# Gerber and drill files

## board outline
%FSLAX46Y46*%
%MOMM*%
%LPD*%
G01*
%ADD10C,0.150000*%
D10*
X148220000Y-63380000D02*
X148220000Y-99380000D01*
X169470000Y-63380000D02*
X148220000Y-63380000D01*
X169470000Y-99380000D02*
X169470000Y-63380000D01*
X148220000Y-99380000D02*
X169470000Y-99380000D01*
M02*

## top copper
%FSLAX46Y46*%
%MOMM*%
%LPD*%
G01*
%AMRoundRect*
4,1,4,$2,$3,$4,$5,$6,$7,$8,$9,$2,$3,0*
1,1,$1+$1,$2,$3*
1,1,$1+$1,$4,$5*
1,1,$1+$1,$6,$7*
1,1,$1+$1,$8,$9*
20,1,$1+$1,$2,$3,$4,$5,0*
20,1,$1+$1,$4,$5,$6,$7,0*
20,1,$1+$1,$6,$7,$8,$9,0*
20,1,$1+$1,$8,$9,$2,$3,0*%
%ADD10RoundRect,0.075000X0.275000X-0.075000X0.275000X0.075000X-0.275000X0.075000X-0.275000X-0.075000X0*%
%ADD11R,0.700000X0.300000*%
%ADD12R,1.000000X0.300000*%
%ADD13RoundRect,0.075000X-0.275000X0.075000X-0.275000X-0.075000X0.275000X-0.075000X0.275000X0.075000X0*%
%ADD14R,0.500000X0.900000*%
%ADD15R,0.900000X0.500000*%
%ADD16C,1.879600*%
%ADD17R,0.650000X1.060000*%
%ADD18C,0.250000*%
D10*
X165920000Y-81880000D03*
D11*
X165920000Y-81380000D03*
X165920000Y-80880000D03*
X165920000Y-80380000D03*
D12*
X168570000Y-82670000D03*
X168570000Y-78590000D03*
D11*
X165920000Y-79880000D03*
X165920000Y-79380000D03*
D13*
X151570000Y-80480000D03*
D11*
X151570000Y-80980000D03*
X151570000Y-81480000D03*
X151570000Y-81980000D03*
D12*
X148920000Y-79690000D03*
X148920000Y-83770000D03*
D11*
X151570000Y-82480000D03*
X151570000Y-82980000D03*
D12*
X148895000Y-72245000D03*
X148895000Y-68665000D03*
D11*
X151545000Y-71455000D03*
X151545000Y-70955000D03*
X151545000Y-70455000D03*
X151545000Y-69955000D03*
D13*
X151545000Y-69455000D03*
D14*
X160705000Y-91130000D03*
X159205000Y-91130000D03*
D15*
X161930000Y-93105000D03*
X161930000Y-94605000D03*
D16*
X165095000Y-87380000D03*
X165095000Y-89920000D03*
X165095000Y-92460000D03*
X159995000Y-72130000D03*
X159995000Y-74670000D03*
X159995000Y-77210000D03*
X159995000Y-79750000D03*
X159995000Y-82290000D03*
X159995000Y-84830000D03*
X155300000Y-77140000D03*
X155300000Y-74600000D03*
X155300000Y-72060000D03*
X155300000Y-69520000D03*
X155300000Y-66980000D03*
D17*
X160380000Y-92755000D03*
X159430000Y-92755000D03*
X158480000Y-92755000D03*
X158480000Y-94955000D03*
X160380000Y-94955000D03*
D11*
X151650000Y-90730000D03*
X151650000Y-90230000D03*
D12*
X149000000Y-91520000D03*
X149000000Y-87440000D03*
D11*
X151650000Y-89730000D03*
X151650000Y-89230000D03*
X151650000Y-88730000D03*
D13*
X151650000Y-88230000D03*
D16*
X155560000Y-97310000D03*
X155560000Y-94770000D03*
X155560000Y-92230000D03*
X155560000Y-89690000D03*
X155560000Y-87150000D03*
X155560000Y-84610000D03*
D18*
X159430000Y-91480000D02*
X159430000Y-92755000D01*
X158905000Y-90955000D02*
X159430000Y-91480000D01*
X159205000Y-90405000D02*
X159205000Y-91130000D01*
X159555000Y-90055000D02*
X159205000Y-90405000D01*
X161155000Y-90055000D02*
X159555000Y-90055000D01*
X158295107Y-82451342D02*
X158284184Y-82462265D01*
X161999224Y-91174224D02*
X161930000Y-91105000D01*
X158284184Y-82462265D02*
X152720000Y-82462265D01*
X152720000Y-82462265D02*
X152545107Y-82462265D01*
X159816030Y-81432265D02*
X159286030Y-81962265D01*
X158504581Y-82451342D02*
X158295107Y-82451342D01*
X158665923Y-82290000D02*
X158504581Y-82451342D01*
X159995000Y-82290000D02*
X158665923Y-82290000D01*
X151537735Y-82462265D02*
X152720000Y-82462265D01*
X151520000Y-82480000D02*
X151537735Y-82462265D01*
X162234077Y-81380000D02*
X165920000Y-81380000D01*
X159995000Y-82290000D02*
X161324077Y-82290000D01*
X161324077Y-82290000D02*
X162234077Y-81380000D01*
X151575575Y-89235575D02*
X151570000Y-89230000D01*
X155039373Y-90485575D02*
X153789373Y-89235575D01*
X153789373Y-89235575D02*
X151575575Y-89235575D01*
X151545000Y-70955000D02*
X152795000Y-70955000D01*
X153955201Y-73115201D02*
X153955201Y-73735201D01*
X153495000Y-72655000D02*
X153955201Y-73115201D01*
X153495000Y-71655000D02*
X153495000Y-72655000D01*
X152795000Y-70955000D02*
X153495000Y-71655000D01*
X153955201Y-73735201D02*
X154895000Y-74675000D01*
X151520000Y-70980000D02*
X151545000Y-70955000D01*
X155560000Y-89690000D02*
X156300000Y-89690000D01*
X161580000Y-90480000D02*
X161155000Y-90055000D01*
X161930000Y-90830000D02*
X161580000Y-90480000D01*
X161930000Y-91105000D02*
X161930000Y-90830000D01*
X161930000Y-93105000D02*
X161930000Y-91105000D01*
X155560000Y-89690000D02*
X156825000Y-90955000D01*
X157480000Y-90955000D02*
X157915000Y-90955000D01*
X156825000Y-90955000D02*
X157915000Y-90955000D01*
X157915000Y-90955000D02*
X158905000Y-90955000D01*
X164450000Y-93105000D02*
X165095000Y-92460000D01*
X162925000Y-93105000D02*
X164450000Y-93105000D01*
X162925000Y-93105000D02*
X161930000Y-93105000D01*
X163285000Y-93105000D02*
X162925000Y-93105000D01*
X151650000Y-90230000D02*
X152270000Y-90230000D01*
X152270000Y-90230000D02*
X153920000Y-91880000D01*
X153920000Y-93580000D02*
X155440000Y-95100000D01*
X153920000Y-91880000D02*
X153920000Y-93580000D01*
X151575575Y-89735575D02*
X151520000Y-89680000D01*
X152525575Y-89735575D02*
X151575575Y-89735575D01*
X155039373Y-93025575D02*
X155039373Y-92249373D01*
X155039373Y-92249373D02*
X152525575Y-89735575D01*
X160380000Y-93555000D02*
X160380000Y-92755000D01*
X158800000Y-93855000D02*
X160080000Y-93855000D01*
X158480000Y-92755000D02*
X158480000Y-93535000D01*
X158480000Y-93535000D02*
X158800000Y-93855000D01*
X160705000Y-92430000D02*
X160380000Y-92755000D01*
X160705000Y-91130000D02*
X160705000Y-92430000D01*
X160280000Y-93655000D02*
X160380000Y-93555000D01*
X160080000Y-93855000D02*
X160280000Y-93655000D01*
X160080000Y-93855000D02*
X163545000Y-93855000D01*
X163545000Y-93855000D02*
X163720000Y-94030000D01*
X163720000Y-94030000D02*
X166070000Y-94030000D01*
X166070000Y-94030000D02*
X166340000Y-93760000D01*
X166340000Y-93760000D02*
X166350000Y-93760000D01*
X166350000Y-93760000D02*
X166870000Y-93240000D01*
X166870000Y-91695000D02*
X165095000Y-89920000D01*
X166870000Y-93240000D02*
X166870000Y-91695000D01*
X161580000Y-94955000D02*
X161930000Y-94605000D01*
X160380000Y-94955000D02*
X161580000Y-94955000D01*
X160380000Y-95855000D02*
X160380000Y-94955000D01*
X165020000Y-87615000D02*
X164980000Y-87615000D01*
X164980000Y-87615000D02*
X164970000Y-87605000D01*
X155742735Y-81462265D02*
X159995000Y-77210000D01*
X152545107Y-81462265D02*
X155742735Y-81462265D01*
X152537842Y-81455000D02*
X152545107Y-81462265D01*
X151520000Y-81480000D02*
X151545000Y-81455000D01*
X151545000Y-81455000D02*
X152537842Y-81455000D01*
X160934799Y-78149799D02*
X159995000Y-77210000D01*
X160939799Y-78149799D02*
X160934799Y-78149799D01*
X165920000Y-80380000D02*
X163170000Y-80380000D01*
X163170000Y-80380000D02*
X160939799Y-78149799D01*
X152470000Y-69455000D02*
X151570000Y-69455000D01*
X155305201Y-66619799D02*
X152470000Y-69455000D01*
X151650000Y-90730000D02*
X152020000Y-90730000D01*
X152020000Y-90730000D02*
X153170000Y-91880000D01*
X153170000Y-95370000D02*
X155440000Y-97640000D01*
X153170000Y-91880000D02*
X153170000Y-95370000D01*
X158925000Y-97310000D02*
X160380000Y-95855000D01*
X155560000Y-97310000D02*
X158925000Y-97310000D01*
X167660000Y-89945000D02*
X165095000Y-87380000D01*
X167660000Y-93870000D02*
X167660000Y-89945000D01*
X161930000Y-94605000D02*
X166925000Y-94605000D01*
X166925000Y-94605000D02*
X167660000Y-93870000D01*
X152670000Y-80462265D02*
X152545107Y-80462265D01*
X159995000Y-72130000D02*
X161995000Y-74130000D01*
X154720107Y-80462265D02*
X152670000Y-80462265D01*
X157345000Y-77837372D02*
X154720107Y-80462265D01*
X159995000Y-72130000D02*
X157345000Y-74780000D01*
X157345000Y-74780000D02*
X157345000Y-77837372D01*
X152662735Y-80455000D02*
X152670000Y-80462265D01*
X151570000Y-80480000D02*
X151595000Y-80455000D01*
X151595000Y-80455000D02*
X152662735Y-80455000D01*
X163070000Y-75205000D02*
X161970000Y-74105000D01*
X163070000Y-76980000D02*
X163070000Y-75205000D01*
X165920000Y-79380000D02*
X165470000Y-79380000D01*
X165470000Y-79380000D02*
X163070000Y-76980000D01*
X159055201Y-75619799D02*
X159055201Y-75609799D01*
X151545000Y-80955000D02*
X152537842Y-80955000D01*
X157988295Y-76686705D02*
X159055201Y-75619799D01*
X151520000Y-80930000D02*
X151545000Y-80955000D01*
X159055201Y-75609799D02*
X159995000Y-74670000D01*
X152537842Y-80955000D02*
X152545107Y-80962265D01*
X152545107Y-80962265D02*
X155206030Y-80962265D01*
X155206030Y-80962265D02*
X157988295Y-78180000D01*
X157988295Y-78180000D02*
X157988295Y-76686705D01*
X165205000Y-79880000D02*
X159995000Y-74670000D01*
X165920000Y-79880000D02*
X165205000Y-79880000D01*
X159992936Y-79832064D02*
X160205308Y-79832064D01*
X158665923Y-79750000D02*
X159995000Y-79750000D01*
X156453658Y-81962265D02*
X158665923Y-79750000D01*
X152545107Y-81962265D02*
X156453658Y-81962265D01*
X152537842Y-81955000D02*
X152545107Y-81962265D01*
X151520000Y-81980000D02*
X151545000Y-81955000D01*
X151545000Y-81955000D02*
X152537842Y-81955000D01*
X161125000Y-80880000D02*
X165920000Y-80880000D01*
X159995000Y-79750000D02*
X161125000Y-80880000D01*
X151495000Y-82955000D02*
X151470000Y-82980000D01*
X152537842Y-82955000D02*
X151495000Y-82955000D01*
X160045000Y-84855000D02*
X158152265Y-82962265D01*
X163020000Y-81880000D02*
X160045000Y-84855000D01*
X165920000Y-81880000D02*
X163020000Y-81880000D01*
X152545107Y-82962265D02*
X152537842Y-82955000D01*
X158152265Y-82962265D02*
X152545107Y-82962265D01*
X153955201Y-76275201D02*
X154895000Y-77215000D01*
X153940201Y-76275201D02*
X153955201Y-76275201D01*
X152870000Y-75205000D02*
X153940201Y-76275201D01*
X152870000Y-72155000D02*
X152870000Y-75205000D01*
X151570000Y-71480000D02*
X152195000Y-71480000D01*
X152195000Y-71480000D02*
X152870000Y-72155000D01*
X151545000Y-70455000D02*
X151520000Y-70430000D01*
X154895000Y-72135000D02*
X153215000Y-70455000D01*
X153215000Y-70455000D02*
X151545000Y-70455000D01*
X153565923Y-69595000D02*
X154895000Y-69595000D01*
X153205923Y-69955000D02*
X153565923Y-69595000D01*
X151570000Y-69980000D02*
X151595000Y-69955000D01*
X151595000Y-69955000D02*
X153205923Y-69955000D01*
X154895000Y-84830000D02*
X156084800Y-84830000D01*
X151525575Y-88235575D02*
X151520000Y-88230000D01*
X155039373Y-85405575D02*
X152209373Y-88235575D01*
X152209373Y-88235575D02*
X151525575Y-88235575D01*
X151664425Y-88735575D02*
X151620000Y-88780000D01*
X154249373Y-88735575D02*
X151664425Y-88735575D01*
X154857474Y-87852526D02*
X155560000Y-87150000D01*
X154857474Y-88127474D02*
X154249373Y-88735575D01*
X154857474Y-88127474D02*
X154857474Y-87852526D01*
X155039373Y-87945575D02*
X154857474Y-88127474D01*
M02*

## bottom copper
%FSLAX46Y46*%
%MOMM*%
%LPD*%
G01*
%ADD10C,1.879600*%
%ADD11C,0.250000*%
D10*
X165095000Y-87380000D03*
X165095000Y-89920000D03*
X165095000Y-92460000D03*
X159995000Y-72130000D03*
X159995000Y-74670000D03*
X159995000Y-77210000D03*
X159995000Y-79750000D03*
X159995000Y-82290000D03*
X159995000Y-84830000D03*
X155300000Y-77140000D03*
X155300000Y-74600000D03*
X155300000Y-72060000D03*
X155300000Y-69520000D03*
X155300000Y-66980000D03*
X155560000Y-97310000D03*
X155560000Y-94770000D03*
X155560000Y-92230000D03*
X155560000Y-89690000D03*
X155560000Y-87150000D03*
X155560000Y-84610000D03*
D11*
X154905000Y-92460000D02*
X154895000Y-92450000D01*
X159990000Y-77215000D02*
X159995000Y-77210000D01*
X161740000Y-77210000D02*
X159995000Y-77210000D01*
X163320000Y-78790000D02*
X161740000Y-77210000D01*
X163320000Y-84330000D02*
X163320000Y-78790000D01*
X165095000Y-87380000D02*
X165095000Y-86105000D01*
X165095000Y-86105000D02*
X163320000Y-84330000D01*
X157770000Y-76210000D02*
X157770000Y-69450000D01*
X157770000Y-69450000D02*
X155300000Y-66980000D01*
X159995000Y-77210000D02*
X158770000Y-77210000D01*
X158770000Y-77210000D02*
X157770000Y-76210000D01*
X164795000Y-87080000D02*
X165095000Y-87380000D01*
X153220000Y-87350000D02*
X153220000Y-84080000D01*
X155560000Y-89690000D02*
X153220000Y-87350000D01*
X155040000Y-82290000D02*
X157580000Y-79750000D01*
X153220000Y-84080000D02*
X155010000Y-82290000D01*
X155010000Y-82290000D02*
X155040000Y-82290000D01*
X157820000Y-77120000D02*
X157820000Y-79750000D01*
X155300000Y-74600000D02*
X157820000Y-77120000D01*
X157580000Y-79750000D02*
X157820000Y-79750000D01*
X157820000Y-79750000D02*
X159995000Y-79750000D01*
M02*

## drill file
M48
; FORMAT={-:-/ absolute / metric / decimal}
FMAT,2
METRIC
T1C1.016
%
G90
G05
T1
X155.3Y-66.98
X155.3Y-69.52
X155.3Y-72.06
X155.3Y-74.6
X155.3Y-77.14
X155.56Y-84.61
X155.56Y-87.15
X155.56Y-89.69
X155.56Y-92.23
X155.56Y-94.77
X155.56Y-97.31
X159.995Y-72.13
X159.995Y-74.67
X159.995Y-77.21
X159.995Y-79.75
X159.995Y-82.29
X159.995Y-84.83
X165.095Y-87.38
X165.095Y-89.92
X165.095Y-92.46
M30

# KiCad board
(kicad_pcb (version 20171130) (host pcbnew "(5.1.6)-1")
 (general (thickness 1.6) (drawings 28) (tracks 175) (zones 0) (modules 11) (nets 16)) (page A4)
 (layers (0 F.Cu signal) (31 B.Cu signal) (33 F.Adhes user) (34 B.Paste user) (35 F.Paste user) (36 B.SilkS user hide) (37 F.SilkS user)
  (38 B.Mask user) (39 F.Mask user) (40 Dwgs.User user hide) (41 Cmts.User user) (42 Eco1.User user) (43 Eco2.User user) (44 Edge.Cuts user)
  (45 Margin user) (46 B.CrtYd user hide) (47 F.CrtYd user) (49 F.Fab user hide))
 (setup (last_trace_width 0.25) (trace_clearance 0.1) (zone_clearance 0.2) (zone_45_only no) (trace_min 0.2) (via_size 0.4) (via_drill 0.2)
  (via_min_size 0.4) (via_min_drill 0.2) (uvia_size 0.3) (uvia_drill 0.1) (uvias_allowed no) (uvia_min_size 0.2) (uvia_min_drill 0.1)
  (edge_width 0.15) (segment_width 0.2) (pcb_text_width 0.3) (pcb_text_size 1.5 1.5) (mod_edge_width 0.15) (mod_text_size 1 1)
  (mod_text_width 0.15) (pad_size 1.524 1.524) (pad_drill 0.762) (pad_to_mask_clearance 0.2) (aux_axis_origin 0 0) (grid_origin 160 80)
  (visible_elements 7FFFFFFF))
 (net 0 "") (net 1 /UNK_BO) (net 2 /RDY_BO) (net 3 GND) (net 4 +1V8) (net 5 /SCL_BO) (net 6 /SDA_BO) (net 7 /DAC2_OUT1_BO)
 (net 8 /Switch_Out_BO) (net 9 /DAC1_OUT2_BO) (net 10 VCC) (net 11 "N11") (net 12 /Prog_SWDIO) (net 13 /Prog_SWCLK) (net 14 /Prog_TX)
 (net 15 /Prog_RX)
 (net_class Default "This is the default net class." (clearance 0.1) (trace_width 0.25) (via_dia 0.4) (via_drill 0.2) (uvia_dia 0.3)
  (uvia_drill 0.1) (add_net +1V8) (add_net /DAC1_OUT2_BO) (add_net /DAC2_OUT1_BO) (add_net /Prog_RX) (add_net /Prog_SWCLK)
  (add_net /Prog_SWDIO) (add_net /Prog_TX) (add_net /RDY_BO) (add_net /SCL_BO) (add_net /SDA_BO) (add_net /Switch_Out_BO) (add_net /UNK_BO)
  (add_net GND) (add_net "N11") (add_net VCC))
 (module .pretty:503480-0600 (layer F.Cu) (at 165.92 80.63 90) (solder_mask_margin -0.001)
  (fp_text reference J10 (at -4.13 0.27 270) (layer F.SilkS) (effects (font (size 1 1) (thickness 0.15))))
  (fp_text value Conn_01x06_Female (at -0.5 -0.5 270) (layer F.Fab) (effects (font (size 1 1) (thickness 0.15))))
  (pad 1 smd roundrect (at -1.25 0 90) (size 0.3 0.7) (layers F.Cu F.Paste F.Mask) (roundrect_rratio 0.25) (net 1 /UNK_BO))
  (pad 2 smd rect (at -0.75 0 90) (size 0.3 0.7) (layers F.Cu F.Paste F.Mask) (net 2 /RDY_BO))
  (pad 3 smd rect (at -0.25 0 90) (size 0.3 0.7) (layers F.Cu F.Paste F.Mask) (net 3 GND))
  (pad 4 smd rect (at 0.25 0 90) (size 0.3 0.7) (layers F.Cu F.Paste F.Mask) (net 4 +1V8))
  (pad 0 smd rect (at -2.04 2.65 90) (size 0.3 1) (layers F.Cu F.Paste F.Mask))
  (pad 0 smd rect (at 2.04 2.65 90) (size 0.3 1) (layers F.Cu F.Paste F.Mask))
  (pad 5 smd rect (at 0.75 0 90) (size 0.3 0.7) (layers F.Cu F.Paste F.Mask) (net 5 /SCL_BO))
  (pad 6 smd rect (at 1.25 0 90) (size 0.3 0.7) (layers F.Cu F.Paste F.Mask) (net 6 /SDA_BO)))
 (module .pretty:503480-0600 (layer F.Cu) (at 151.57 81.73 270) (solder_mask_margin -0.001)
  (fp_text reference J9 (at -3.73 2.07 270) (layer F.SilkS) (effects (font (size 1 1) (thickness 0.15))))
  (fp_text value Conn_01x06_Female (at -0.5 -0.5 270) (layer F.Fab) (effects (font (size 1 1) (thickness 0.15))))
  (pad 1 smd roundrect (at -1.25 0 270) (size 0.3 0.7) (layers F.Cu F.Paste F.Mask) (roundrect_rratio 0.25) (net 6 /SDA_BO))
  (pad 2 smd rect (at -0.75 0 270) (size 0.3 0.7) (layers F.Cu F.Paste F.Mask) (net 5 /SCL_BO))
  (pad 3 smd rect (at -0.25 0 270) (size 0.3 0.7) (layers F.Cu F.Paste F.Mask) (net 4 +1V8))
  (pad 4 smd rect (at 0.25 0 270) (size 0.3 0.7) (layers F.Cu F.Paste F.Mask) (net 3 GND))
  (pad 0 smd rect (at -2.04 2.65 270) (size 0.3 1) (layers F.Cu F.Paste F.Mask))
  (pad 0 smd rect (at 2.04 2.65 270) (size 0.3 1) (layers F.Cu F.Paste F.Mask))
  (pad 5 smd rect (at 0.75 0 270) (size 0.3 0.7) (layers F.Cu F.Paste F.Mask) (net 2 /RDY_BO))
  (pad 6 smd rect (at 1.25 0 270) (size 0.3 0.7) (layers F.Cu F.Paste F.Mask) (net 1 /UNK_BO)))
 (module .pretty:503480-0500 (layer F.Cu) (at 151.545 70.455 270) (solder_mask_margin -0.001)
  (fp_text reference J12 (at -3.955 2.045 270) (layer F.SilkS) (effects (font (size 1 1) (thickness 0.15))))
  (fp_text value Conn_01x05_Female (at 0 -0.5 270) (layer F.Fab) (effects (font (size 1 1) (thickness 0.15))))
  (pad 0 smd rect (at 1.79 2.65 270) (size 0.3 1) (layers F.Cu F.Paste F.Mask))
  (pad 0 smd rect (at -1.79 2.65 270) (size 0.3 1) (layers F.Cu F.Paste F.Mask))
  (pad 5 smd rect (at 1 0 270) (size 0.3 0.7) (layers F.Cu F.Paste F.Mask) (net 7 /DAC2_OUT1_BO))
  (pad 4 smd rect (at 0.5 0 270) (size 0.3 0.7) (layers F.Cu F.Paste F.Mask) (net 3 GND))
  (pad 3 smd rect (at 0 0 270) (size 0.3 0.7) (layers F.Cu F.Paste F.Mask) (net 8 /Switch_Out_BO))
  (pad 2 smd rect (at -0.5 0 270) (size 0.3 0.7) (layers F.Cu F.Paste F.Mask) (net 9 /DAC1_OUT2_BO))
  (pad 1 smd roundrect (at -1 0 270) (size 0.3 0.7) (layers F.Cu F.Paste F.Mask) (roundrect_rratio 0.25) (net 4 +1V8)))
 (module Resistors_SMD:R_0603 (layer F.Cu) (at 159.955 91.13)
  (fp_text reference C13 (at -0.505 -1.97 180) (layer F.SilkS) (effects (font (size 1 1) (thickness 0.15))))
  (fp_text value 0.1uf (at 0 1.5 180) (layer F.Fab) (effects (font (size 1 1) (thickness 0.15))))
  (pad 2 smd rect (at 0.75 0) (size 0.5 0.9) (layers F.Cu F.Paste F.Mask) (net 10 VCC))
  (pad 1 smd rect (at -0.75 0) (size 0.5 0.9) (layers F.Cu F.Paste F.Mask) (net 3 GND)))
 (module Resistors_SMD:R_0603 (layer F.Cu) (at 161.93 93.855 270)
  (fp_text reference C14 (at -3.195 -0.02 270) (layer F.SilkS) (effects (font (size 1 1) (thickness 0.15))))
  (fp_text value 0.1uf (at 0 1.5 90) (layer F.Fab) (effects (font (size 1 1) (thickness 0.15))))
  (pad 1 smd rect (at -0.75 0 270) (size 0.5 0.9) (layers F.Cu F.Paste F.Mask) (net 3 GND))
  (pad 2 smd rect (at 0.75 0 270) (size 0.5 0.9) (layers F.Cu F.Paste F.Mask) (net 4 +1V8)))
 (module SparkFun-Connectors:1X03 (layer F.Cu) (at 165.095 87.38 270)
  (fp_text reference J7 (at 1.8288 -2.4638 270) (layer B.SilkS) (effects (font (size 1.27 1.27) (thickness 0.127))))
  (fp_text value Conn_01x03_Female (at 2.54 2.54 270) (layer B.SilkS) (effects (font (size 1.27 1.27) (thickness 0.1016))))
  (pad 1 thru_hole circle (at 0 0 270) (size 1.8796 1.8796) (drill 1.016) (layers F&B.Cu F.Paste F.SilkS F.Mask) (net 4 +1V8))
  (pad 2 thru_hole circle (at 2.54 0 270) (size 1.8796 1.8796) (drill 1.016) (layers F&B.Cu F.Paste F.SilkS F.Mask) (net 10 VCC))
  (pad 3 thru_hole circle (at 5.08 0 270) (size 1.8796 1.8796) (drill 1.016) (layers F&B.Cu F.Paste F.SilkS F.Mask) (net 3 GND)))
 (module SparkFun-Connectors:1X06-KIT (layer F.Cu) (at 159.995 72.13 270)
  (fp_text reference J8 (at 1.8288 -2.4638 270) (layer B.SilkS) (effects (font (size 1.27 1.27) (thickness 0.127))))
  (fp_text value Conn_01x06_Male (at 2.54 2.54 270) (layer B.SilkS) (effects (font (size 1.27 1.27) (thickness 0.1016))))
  (pad 1 thru_hole circle (at 0 0 270) (size 1.8796 1.8796) (drill 1.016) (layers F&B.Cu F.Paste F.SilkS F.Mask) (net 6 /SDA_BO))
  (pad 2 thru_hole circle (at 2.54 0 270) (size 1.8796 1.8796) (drill 1.016) (layers F&B.Cu F.Paste F.SilkS F.Mask) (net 5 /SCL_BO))
  (pad 3 thru_hole circle (at 5.08 0 270) (size 1.8796 1.8796) (drill 1.016) (layers F&B.Cu F.Paste F.SilkS F.Mask) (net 4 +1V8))
  (pad 4 thru_hole circle (at 7.62 0 270) (size 1.8796 1.8796) (drill 1.016) (layers F&B.Cu F.Paste F.SilkS F.Mask) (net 3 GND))
  (pad 5 thru_hole circle (at 10.16 0 270) (size 1.8796 1.8796) (drill 1.016) (layers F&B.Cu F.Paste F.SilkS F.Mask) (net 2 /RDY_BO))
  (pad 6 thru_hole circle (at 12.7 0 270) (size 1.8796 1.8796) (drill 1.016) (layers F&B.Cu F.Paste F.SilkS F.Mask) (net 1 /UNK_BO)))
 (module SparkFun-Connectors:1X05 (layer F.Cu) (at 155.3 77.14 90)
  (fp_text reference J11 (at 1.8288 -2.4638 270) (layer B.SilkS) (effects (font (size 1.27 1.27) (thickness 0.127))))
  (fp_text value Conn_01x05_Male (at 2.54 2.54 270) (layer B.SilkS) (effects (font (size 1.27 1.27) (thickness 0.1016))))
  (pad 1 thru_hole circle (at 0 0 90) (size 1.8796 1.8796) (drill 1.016) (layers F&B.Cu F.Paste F.SilkS F.Mask) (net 7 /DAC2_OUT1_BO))
  (pad 2 thru_hole circle (at 2.54 0 90) (size 1.8796 1.8796) (drill 1.016) (layers F&B.Cu F.Paste F.SilkS F.Mask) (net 3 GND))
  (pad 3 thru_hole circle (at 5.08 0 90) (size 1.8796 1.8796) (drill 1.016) (layers F&B.Cu F.Paste F.SilkS F.Mask) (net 8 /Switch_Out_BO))
  (pad 4 thru_hole circle (at 7.62 0 90) (size 1.8796 1.8796) (drill 1.016) (layers F&B.Cu F.Paste F.SilkS F.Mask) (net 9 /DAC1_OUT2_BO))
  (pad 5 thru_hole circle (at 10.16 0 90) (size 1.8796 1.8796) (drill 1.016) (layers F&B.Cu F.Paste F.SilkS F.Mask) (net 4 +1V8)))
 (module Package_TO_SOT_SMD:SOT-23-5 (layer F.Cu) (at 159.43 93.855 270) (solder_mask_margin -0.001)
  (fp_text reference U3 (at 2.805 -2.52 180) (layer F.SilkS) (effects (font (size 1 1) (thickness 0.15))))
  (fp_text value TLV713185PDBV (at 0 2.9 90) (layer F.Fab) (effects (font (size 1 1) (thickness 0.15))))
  (pad 1 smd rect (at -1.1 -0.95 270) (size 1.06 0.65) (layers F.Cu F.Paste F.Mask) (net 10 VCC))
  (pad 2 smd rect (at -1.1 0 270) (size 1.06 0.65) (layers F.Cu F.Paste F.Mask) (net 3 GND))
  (pad 3 smd rect (at -1.1 0.95 270) (size 1.06 0.65) (layers F.Cu F.Paste F.Mask) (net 10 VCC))
  (pad 4 smd rect (at 1.1 0.95 270) (size 1.06 0.65) (layers F.Cu F.Paste F.Mask) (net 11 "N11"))
  (pad 5 smd rect (at 1.1 -0.95 270) (size 1.06 0.65) (layers F.Cu F.Paste F.Mask) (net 4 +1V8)))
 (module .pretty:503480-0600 (layer F.Cu) (at 151.65 89.48 270) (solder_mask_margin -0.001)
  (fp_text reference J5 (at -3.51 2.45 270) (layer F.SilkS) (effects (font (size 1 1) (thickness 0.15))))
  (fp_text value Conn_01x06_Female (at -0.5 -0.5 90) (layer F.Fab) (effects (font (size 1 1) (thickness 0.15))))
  (pad 6 smd rect (at 1.25 0 270) (size 0.3 0.7) (layers F.Cu F.Paste F.Mask) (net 4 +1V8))
  (pad 5 smd rect (at 0.75 0 270) (size 0.3 0.7) (layers F.Cu F.Paste F.Mask) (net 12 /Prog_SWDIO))
  (pad 0 smd rect (at 2.04 2.65 270) (size 0.3 1) (layers F.Cu F.Paste F.Mask))
  (pad 0 smd rect (at -2.04 2.65 270) (size 0.3 1) (layers F.Cu F.Paste F.Mask))
  (pad 4 smd rect (at 0.25 0 270) (size 0.3 0.7) (layers F.Cu F.Paste F.Mask) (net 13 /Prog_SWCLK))
  (pad 3 smd rect (at -0.25 0 270) (size 0.3 0.7) (layers F.Cu F.Paste F.Mask) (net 3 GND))
  (pad 2 smd rect (at -0.75 0 270) (size 0.3 0.7) (layers F.Cu F.Paste F.Mask) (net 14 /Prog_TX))
  (pad 1 smd roundrect (at -1.25 0 270) (size 0.3 0.7) (layers F.Cu F.Paste F.Mask) (roundrect_rratio 0.25) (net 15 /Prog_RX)))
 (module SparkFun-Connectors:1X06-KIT (layer F.Cu) (at 155.56 97.31 90)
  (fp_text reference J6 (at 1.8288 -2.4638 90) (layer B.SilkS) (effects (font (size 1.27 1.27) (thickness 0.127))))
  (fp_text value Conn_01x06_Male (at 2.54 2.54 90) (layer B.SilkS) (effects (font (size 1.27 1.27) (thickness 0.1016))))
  (pad 1 thru_hole circle (at 0 0 90) (size 1.8796 1.8796) (drill 1.016) (layers F&B.Cu F.Paste F.SilkS F.Mask) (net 4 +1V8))
  (pad 2 thru_hole circle (at 2.54 0 90) (size 1.8796 1.8796) (drill 1.016) (layers F&B.Cu F.Paste F.SilkS F.Mask) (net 12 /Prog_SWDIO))
  (pad 3 thru_hole circle (at 5.08 0 90) (size 1.8796 1.8796) (drill 1.016) (layers F&B.Cu F.Paste F.SilkS F.Mask) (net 13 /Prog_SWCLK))
  (pad 4 thru_hole circle (at 7.62 0 90) (size 1.8796 1.8796) (drill 1.016) (layers F&B.Cu F.Paste F.SilkS F.Mask) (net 3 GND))
  (pad 5 thru_hole circle (at 10.16 0 90) (size 1.8796 1.8796) (drill 1.016) (layers F&B.Cu F.Paste F.SilkS F.Mask) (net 14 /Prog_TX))
  (pad 6 thru_hole circle (at 12.7 0 90) (size 1.8796 1.8796) (drill 1.016) (layers F&B.Cu F.Paste F.SilkS F.Mask) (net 15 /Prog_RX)))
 (gr_line (start 148.22 63.38) (end 148.22 99.38) (layer Edge.Cuts) (width 0.15))
 (gr_line (start 169.47 63.38) (end 148.22 63.38) (layer Edge.Cuts) (width 0.15))
 (gr_line (start 169.47 99.38) (end 169.47 63.38) (layer Edge.Cuts) (width 0.15))
 (gr_line (start 148.22 99.38) (end 169.47 99.38) (layer Edge.Cuts) (width 0.15))
 (segment (start 159.43 91.48) (end 159.43 92.755) (width 0.25) (layer F.Cu) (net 3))
 (segment (start 158.905 90.955) (end 159.43 91.48) (width 0.25) (layer F.Cu) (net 3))
 (segment (start 159.205 90.405) (end 159.205 91.13) (width 0.25) (layer F.Cu) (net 3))
 (segment (start 159.555 90.055) (end 159.205 90.405) (width 0.25) (layer F.Cu) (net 3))
 (segment (start 161.155 90.055) (end 159.555 90.055) (width 0.25) (layer F.Cu) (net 3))
 (segment (start 158.295107 82.451342) (end 158.284184 82.462265) (width 0.25) (layer F.Cu) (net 2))
 (segment (start 161.999224 91.174224) (end 161.93 91.105) (width 0.25) (layer F.Cu) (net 3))
 (segment (start 158.284184 82.462265) (end 152.72 82.462265) (width 0.25) (layer F.Cu) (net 2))
 (segment (start 152.72 82.462265) (end 152.545107 82.462265) (width 0.25) (layer F.Cu) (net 2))
 (segment (start 159.81603 81.432265) (end 159.28603 81.962265) (width 0.25) (layer F.Cu) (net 2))
 (segment (start 158.504581 82.451342) (end 158.295107 82.451342) (width 0.25) (layer F.Cu) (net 2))
 (segment (start 158.665923 82.29) (end 158.504581 82.451342) (width 0.25) (layer F.Cu) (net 2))
 (segment (start 159.995 82.29) (end 158.665923 82.29) (width 0.25) (layer F.Cu) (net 2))
 (segment (start 151.537735 82.462265) (end 152.72 82.462265) (width 0.25) (layer F.Cu) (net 2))
 (segment (start 151.52 82.48) (end 151.537735 82.462265) (width 0.25) (layer F.Cu) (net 2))
 (segment (start 162.234077 81.38) (end 165.92 81.38) (width 0.25) (layer F.Cu) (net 2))
 (segment (start 159.995 82.29) (end 161.324077 82.29) (width 0.25) (layer F.Cu) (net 2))
 (segment (start 161.324077 82.29) (end 162.234077 81.38) (width 0.25) (layer F.Cu) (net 2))
 (segment (start 151.575575 89.235575) (end 151.57 89.23) (width 0.25) (layer F.Cu) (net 3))
 (segment (start 155.039373 90.485575) (end 153.789373 89.235575) (width 0.25) (layer F.Cu) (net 3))
 (segment (start 153.789373 89.235575) (end 151.575575 89.235575) (width 0.25) (layer F.Cu) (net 3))
 (segment (start 151.545 70.955) (end 152.795 70.955) (width 0.25) (layer F.Cu) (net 3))
 (segment (start 153.955201 73.115201) (end 153.955201 73.735201) (width 0.25) (layer F.Cu) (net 3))
 (segment (start 153.495 72.655) (end 153.955201 73.115201) (width 0.25) (layer F.Cu) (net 3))
 (segment (start 153.495 71.655) (end 153.495 72.655) (width 0.25) (layer F.Cu) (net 3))
 (segment (start 152.795 70.955) (end 153.495 71.655) (width 0.25) (layer F.Cu) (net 3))
 (segment (start 153.955201 73.735201) (end 154.895 74.675) (width 0.25) (layer F.Cu) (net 3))
 (segment (start 151.52 70.98) (end 151.545 70.955) (width 0.25) (layer F.Cu) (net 3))
 (segment (start 155.56 89.69) (end 156.3 89.69) (width 0.25) (layer F.Cu) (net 3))
 (segment (start 161.58 90.48) (end 161.155 90.055) (width 0.25) (layer F.Cu) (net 3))
 (segment (start 161.93 90.83) (end 161.58 90.48) (width 0.25) (layer F.Cu) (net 3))
 (segment (start 161.93 91.105) (end 161.93 90.83) (width 0.25) (layer F.Cu) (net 3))
 (segment (start 161.93 93.105) (end 161.93 91.105) (width 0.25) (layer F.Cu) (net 3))
 (segment (start 155.56 89.69) (end 156.825 90.955) (width 0.25) (layer F.Cu) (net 3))
 (segment (start 157.48 90.955) (end 157.915 90.955) (width 0.25) (layer F.Cu) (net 3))
 (segment (start 156.825 90.955) (end 157.915 90.955) (width 0.25) (layer F.Cu) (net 3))
 (segment (start 157.915 90.955) (end 158.905 90.955) (width 0.25) (layer F.Cu) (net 3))
 (segment (start 164.45 93.105) (end 165.095 92.46) (width 0.25) (layer F.Cu) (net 3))
 (segment (start 162.925 93.105) (end 164.45 93.105) (width 0.25) (layer F.Cu) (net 3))
 (segment (start 162.925 93.105) (end 161.93 93.105) (width 0.25) (layer F.Cu) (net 3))
 (segment (start 163.285 93.105) (end 162.925 93.105) (width 0.25) (layer F.Cu) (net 3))
 (segment (start 151.65 90.23) (end 152.27 90.23) (width 0.25) (layer F.Cu) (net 12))
 (segment (start 152.27 90.23) (end 153.92 91.88) (width 0.25) (layer F.Cu) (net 12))
 (segment (start 153.92 93.58) (end 155.44 95.1) (width 0.25) (layer F.Cu) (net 12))
 (segment (start 153.92 91.88) (end 153.92 93.58) (width 0.25) (layer F.Cu) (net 12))
 (segment (start 154.905 92.46) (end 154.895 92.45) (width 0.25) (layer B.Cu) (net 13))
 (segment (start 151.575575 89.735575) (end 151.52 89.68) (width 0.25) (layer F.Cu) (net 13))
 (segment (start 152.525575 89.735575) (end 151.575575 89.735575) (width 0.25) (layer F.Cu) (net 13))
 (segment (start 155.039373 93.025575) (end 155.039373 92.249373) (width 0.25) (layer F.Cu) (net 13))
 (segment (start 155.039373 92.249373) (end 152.525575 89.735575) (width 0.25) (layer F.Cu) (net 13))
 (segment (start 160.38 93.555) (end 160.38 92.755) (width 0.25) (layer F.Cu) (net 10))
 (segment (start 158.8 93.855) (end 160.08 93.855) (width 0.25) (layer F.Cu) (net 10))
 (segment (start 158.48 92.755) (end 158.48 93.535) (width 0.25) (layer F.Cu) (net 10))
 (segment (start 158.48 93.535) (end 158.8 93.855) (width 0.25) (layer F.Cu) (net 10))
 (segment (start 160.705 92.43) (end 160.38 92.755) (width 0.25) (layer F.Cu) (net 10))
 (segment (start 160.705 91.13) (end 160.705 92.43) (width 0.25) (layer F.Cu) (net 10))
 (segment (start 160.28 93.655) (end 160.38 93.555) (width 0.25) (layer F.Cu) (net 10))
 (segment (start 160.08 93.855) (end 160.28 93.655) (width 0.25) (layer F.Cu) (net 10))
 (segment (start 160.08 93.855) (end 163.545 93.855) (width 0.25) (layer F.Cu) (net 10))
 (segment (start 163.545 93.855) (end 163.72 94.03) (width 0.25) (layer F.Cu) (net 10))
 (segment (start 163.72 94.03) (end 166.07 94.03) (width 0.25) (layer F.Cu) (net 10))
 (segment (start 166.07 94.03) (end 166.34 93.76) (width 0.25) (layer F.Cu) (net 10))
 (segment (start 166.34 93.76) (end 166.35 93.76) (width 0.25) (layer F.Cu) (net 10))
 (segment (start 166.35 93.76) (end 166.87 93.24) (width 0.25) (layer F.Cu) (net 10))
 (segment (start 166.87 91.695) (end 165.095 89.92) (width 0.25) (layer F.Cu) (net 10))
 (segment (start 166.87 93.24) (end 166.87 91.695) (width 0.25) (layer F.Cu) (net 10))
 (segment (start 161.58 94.955) (end 161.93 94.605) (width 0.25) (layer F.Cu) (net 4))
 (segment (start 160.38 94.955) (end 161.58 94.955) (width 0.25) (layer F.Cu) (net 4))
 (segment (start 160.38 95.855) (end 160.38 94.955) (width 0.25) (layer F.Cu) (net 4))
 (segment (start 165.02 87.615) (end 164.98 87.615) (width 0.25) (layer F.Cu) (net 4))
 (segment (start 164.98 87.615) (end 164.97 87.605) (width 0.25) (layer F.Cu) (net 4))
 (segment (start 155.742735 81.462265) (end 159.995 77.21) (width 0.25) (layer F.Cu) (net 4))
 (segment (start 152.545107 81.462265) (end 155.742735 81.462265) (width 0.25) (layer F.Cu) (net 4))
 (segment (start 152.537842 81.455) (end 152.545107 81.462265) (width 0.25) (layer F.Cu) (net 4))
 (segment (start 151.52 81.48) (end 151.545 81.455) (width 0.25) (layer F.Cu) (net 4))
 (segment (start 151.545 81.455) (end 152.537842 81.455) (width 0.25) (layer F.Cu) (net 4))
 (segment (start 159.99 77.215) (end 159.995 77.21) (width 0.25) (layer B.Cu) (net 4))
 (segment (start 160.934799 78.149799) (end 159.995 77.21) (width 0.25) (layer F.Cu) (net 4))
 (segment (start 160.939799 78.149799) (end 160.934799 78.149799) (width 0.25) (layer F.Cu) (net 4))
 (segment (start 165.92 80.38) (end 163.17 80.38) (width 0.25) (layer F.Cu) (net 4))
 (segment (start 163.17 80.38) (end 160.939799 78.149799) (width 0.25) (layer F.Cu) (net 4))
 (segment (start 152.47 69.455) (end 151.57 69.455) (width 0.25) (layer F.Cu) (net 4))
 (segment (start 155.305201 66.619799) (end 152.47 69.455) (width 0.25) (layer F.Cu) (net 4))
 (segment (start 161.74 77.21) (end 159.995 77.21) (width 0.25) (layer B.Cu) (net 4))
 (segment (start 163.32 78.79) (end 161.74 77.21) (width 0.25) (layer B.Cu) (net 4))
 (segment (start 163.32 84.33) (end 163.32 78.79) (width 0.25) (layer B.Cu) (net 4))
 (segment (start 165.095 87.38) (end 165.095 86.105) (width 0.25) (layer B.Cu) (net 4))
 (segment (start 165.095 86.105) (end 163.32 84.33) (width 0.25) (layer B.Cu) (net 4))
 (segment (start 157.77 76.21) (end 157.77 69.45) (width 0.25) (layer B.Cu) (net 4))
 (segment (start 157.77 69.45) (end 155.3 66.98) (width 0.25) (layer B.Cu) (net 4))
 (segment (start 159.995 77.21) (end 158.77 77.21) (width 0.25) (layer B.Cu) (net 4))
 (segment (start 158.77 77.21) (end 157.77 76.21) (width 0.25) (layer B.Cu) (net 4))
 (segment (start 164.795 87.08) (end 165.095 87.38) (width 0.25) (layer B.Cu) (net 4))
 (segment (start 151.65 90.73) (end 152.02 90.73) (width 0.25) (layer F.Cu) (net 4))
 (segment (start 152.02 90.73) (end 153.17 91.88) (width 0.25) (layer F.Cu) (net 4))
 (segment (start 153.17 95.37) (end 155.44 97.64) (width 0.25) (layer F.Cu) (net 4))
 (segment (start 153.17 91.88) (end 153.17 95.37) (width 0.25) (layer F.Cu) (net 4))
 (segment (start 158.925 97.31) (end 160.38 95.855) (width 0.25) (layer F.Cu) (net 4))
 (segment (start 155.56 97.31) (end 158.925 97.31) (width 0.25) (layer F.Cu) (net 4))
 (segment (start 167.66 89.945) (end 165.095 87.38) (width 0.25) (layer F.Cu) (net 4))
 (segment (start 167.66 93.87) (end 167.66 89.945) (width 0.25) (layer F.Cu) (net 4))
 (segment (start 161.93 94.605) (end 166.925 94.605) (width 0.25) (layer F.Cu) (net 4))
 (segment (start 166.925 94.605) (end 167.66 93.87) (width 0.25) (layer F.Cu) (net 4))
 (segment (start 152.67 80.462265) (end 152.545107 80.462265) (width 0.25) (layer F.Cu) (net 6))
 (segment (start 159.995 72.13) (end 161.995 74.13) (width 0.25) (layer F.Cu) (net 6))
 (segment (start 154.720107 80.462265) (end 152.67 80.462265) (width 0.25) (layer F.Cu) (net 6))
 (segment (start 157.345 77.837372) (end 154.720107 80.462265) (width 0.25) (layer F.Cu) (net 6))
 (segment (start 159.995 72.13) (end 157.345 74.78) (width 0.25) (layer F.Cu) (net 6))
 (segment (start 157.345 74.78) (end 157.345 77.837372) (width 0.25) (layer F.Cu) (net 6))
 (segment (start 152.662735 80.455) (end 152.67 80.462265) (width 0.25) (layer F.Cu) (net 6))
 (segment (start 151.57 80.48) (end 151.595 80.455) (width 0.25) (layer F.Cu) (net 6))
 (segment (start 151.595 80.455) (end 152.662735 80.455) (width 0.25) (layer F.Cu) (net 6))
 (segment (start 163.07 75.205) (end 161.97 74.105) (width 0.25) (layer F.Cu) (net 6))
 (segment (start 163.07 76.98) (end 163.07 75.205) (width 0.25) (layer F.Cu) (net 6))
 (segment (start 165.92 79.38) (end 165.47 79.38) (width 0.25) (layer F.Cu) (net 6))
 (segment (start 165.47 79.38) (end 163.07 76.98) (width 0.25) (layer F.Cu) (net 6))
 (segment (start 159.055201 75.619799) (end 159.055201 75.609799) (width 0.25) (layer F.Cu) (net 5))
 (segment (start 151.545 80.955) (end 152.537842 80.955) (width 0.25) (layer F.Cu) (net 5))
 (segment (start 157.988295 76.686705) (end 159.055201 75.619799) (width 0.25) (layer F.Cu) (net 5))
 (segment (start 151.52 80.93) (end 151.545 80.955) (width 0.25) (layer F.Cu) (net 5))
 (segment (start 159.055201 75.609799) (end 159.995 74.67) (width 0.25) (layer F.Cu) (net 5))
 (segment (start 152.537842 80.955) (end 152.545107 80.962265) (width 0.25) (layer F.Cu) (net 5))
 (segment (start 152.545107 80.962265) (end 155.20603 80.962265) (width 0.25) (layer F.Cu) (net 5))
 (segment (start 155.20603 80.962265) (end 157.988295 78.18) (width 0.25) (layer F.Cu) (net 5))
 (segment (start 157.988295 78.18) (end 157.988295 76.686705) (width 0.25) (layer F.Cu) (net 5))
 (segment (start 165.205 79.88) (end 159.995 74.67) (width 0.25) (layer F.Cu) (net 5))
 (segment (start 165.92 79.88) (end 165.205 79.88) (width 0.25) (layer F.Cu) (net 5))
 (segment (start 159.992936 79.832064) (end 160.205308 79.832064) (width 0.25) (layer F.Cu) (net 3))
 (segment (start 158.665923 79.75) (end 159.995 79.75) (width 0.25) (layer F.Cu) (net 3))
 (segment (start 156.453658 81.962265) (end 158.665923 79.75) (width 0.25) (layer F.Cu) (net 3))
 (segment (start 152.545107 81.962265) (end 156.453658 81.962265) (width 0.25) (layer F.Cu) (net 3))
 (segment (start 152.537842 81.955) (end 152.545107 81.962265) (width 0.25) (layer F.Cu) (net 3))
 (segment (start 151.52 81.98) (end 151.545 81.955) (width 0.25) (layer F.Cu) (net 3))
 (segment (start 151.545 81.955) (end 152.537842 81.955) (width 0.25) (layer F.Cu) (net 3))
 (segment (start 161.125 80.88) (end 165.92 80.88) (width 0.25) (layer F.Cu) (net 3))
 (segment (start 159.995 79.75) (end 161.125 80.88) (width 0.25) (layer F.Cu) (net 3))
 (segment (start 153.22 87.35) (end 153.22 84.08) (width 0.25) (layer B.Cu) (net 3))
 (segment (start 155.56 89.69) (end 153.22 87.35) (width 0.25) (layer B.Cu) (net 3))
 (segment (start 155.04 82.29) (end 157.58 79.75) (width 0.25) (layer B.Cu) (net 3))
 (segment (start 153.22 84.08) (end 155.01 82.29) (width 0.25) (layer B.Cu) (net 3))
 (segment (start 155.01 82.29) (end 155.04 82.29) (width 0.25) (layer B.Cu) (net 3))
 (segment (start 157.82 77.12) (end 157.82 79.75) (width 0.25) (layer B.Cu) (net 3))
 (segment (start 155.3 74.6) (end 157.82 77.12) (width 0.25) (layer B.Cu) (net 3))
 (segment (start 157.58 79.75) (end 157.82 79.75) (width 0.25) (layer B.Cu) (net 3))
 (segment (start 157.82 79.75) (end 159.995 79.75) (width 0.25) (layer B.Cu) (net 3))
 (segment (start 151.495 82.955) (end 151.47 82.98) (width 0.25) (layer F.Cu) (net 1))
 (segment (start 152.537842 82.955) (end 151.495 82.955) (width 0.25) (layer F.Cu) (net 1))
 (segment (start 160.045 84.855) (end 158.152265 82.962265) (width 0.25) (layer F.Cu) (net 1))
 (segment (start 163.02 81.88) (end 160.045 84.855) (width 0.25) (layer F.Cu) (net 1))
 (segment (start 165.92 81.88) (end 163.02 81.88) (width 0.25) (layer F.Cu) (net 1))
 (segment (start 152.545107 82.962265) (end 152.537842 82.955) (width 0.25) (layer F.Cu) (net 1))
 (segment (start 158.152265 82.962265) (end 152.545107 82.962265) (width 0.25) (layer F.Cu) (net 1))
 (segment (start 153.955201 76.275201) (end 154.895 77.215) (width 0.25) (layer F.Cu) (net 7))
 (segment (start 153.940201 76.275201) (end 153.955201 76.275201) (width 0.25) (layer F.Cu) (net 7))
 (segment (start 152.87 75.205) (end 153.940201 76.275201) (width 0.25) (layer F.Cu) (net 7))
 (segment (start 152.87 72.155) (end 152.87 75.205) (width 0.25) (layer F.Cu) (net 7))
 (segment (start 151.57 71.48) (end 152.195 71.48) (width 0.25) (layer F.Cu) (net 7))
 (segment (start 152.195 71.48) (end 152.87 72.155) (width 0.25) (layer F.Cu) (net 7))
 (segment (start 151.545 70.455) (end 151.52 70.43) (width 0.25) (layer F.Cu) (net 8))
 (segment (start 154.895 72.135) (end 153.215 70.455) (width 0.25) (layer F.Cu) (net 8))
 (segment (start 153.215 70.455) (end 151.545 70.455) (width 0.25) (layer F.Cu) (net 8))
 (segment (start 153.565923 69.595) (end 154.895 69.595) (width 0.25) (layer F.Cu) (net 9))
 (segment (start 153.205923 69.955) (end 153.565923 69.595) (width 0.25) (layer F.Cu) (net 9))
 (segment (start 151.57 69.98) (end 151.595 69.955) (width 0.25) (layer F.Cu) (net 9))
 (segment (start 151.595 69.955) (end 153.205923 69.955) (width 0.25) (layer F.Cu) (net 9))
 (segment (start 154.895 84.83) (end 156.0848 84.83) (width 0.25) (layer F.Cu) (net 15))
 (segment (start 151.525575 88.235575) (end 151.52 88.23) (width 0.25) (layer F.Cu) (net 15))
 (segment (start 155.039373 85.405575) (end 152.209373 88.235575) (width 0.25) (layer F.Cu) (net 15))
 (segment (start 152.209373 88.235575) (end 151.525575 88.235575) (width 0.25) (layer F.Cu) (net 15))
 (segment (start 151.664425 88.735575) (end 151.62 88.78) (width 0.25) (layer F.Cu) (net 14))
 (segment (start 154.249373 88.735575) (end 151.664425 88.735575) (width 0.25) (layer F.Cu) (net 14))
 (segment (start 154.857474 87.852526) (end 155.56 87.15) (width 0.25) (layer F.Cu) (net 14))
 (segment (start 154.857474 88.127474) (end 154.249373 88.735575) (width 0.25) (layer F.Cu) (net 14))
 (segment (start 154.857474 88.127474) (end 154.857474 87.852526) (width 0.25) (layer F.Cu) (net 14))
 (segment (start 155.039373 87.945575) (end 154.857474 88.127474) (width 0.25) (layer F.Cu) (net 14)))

